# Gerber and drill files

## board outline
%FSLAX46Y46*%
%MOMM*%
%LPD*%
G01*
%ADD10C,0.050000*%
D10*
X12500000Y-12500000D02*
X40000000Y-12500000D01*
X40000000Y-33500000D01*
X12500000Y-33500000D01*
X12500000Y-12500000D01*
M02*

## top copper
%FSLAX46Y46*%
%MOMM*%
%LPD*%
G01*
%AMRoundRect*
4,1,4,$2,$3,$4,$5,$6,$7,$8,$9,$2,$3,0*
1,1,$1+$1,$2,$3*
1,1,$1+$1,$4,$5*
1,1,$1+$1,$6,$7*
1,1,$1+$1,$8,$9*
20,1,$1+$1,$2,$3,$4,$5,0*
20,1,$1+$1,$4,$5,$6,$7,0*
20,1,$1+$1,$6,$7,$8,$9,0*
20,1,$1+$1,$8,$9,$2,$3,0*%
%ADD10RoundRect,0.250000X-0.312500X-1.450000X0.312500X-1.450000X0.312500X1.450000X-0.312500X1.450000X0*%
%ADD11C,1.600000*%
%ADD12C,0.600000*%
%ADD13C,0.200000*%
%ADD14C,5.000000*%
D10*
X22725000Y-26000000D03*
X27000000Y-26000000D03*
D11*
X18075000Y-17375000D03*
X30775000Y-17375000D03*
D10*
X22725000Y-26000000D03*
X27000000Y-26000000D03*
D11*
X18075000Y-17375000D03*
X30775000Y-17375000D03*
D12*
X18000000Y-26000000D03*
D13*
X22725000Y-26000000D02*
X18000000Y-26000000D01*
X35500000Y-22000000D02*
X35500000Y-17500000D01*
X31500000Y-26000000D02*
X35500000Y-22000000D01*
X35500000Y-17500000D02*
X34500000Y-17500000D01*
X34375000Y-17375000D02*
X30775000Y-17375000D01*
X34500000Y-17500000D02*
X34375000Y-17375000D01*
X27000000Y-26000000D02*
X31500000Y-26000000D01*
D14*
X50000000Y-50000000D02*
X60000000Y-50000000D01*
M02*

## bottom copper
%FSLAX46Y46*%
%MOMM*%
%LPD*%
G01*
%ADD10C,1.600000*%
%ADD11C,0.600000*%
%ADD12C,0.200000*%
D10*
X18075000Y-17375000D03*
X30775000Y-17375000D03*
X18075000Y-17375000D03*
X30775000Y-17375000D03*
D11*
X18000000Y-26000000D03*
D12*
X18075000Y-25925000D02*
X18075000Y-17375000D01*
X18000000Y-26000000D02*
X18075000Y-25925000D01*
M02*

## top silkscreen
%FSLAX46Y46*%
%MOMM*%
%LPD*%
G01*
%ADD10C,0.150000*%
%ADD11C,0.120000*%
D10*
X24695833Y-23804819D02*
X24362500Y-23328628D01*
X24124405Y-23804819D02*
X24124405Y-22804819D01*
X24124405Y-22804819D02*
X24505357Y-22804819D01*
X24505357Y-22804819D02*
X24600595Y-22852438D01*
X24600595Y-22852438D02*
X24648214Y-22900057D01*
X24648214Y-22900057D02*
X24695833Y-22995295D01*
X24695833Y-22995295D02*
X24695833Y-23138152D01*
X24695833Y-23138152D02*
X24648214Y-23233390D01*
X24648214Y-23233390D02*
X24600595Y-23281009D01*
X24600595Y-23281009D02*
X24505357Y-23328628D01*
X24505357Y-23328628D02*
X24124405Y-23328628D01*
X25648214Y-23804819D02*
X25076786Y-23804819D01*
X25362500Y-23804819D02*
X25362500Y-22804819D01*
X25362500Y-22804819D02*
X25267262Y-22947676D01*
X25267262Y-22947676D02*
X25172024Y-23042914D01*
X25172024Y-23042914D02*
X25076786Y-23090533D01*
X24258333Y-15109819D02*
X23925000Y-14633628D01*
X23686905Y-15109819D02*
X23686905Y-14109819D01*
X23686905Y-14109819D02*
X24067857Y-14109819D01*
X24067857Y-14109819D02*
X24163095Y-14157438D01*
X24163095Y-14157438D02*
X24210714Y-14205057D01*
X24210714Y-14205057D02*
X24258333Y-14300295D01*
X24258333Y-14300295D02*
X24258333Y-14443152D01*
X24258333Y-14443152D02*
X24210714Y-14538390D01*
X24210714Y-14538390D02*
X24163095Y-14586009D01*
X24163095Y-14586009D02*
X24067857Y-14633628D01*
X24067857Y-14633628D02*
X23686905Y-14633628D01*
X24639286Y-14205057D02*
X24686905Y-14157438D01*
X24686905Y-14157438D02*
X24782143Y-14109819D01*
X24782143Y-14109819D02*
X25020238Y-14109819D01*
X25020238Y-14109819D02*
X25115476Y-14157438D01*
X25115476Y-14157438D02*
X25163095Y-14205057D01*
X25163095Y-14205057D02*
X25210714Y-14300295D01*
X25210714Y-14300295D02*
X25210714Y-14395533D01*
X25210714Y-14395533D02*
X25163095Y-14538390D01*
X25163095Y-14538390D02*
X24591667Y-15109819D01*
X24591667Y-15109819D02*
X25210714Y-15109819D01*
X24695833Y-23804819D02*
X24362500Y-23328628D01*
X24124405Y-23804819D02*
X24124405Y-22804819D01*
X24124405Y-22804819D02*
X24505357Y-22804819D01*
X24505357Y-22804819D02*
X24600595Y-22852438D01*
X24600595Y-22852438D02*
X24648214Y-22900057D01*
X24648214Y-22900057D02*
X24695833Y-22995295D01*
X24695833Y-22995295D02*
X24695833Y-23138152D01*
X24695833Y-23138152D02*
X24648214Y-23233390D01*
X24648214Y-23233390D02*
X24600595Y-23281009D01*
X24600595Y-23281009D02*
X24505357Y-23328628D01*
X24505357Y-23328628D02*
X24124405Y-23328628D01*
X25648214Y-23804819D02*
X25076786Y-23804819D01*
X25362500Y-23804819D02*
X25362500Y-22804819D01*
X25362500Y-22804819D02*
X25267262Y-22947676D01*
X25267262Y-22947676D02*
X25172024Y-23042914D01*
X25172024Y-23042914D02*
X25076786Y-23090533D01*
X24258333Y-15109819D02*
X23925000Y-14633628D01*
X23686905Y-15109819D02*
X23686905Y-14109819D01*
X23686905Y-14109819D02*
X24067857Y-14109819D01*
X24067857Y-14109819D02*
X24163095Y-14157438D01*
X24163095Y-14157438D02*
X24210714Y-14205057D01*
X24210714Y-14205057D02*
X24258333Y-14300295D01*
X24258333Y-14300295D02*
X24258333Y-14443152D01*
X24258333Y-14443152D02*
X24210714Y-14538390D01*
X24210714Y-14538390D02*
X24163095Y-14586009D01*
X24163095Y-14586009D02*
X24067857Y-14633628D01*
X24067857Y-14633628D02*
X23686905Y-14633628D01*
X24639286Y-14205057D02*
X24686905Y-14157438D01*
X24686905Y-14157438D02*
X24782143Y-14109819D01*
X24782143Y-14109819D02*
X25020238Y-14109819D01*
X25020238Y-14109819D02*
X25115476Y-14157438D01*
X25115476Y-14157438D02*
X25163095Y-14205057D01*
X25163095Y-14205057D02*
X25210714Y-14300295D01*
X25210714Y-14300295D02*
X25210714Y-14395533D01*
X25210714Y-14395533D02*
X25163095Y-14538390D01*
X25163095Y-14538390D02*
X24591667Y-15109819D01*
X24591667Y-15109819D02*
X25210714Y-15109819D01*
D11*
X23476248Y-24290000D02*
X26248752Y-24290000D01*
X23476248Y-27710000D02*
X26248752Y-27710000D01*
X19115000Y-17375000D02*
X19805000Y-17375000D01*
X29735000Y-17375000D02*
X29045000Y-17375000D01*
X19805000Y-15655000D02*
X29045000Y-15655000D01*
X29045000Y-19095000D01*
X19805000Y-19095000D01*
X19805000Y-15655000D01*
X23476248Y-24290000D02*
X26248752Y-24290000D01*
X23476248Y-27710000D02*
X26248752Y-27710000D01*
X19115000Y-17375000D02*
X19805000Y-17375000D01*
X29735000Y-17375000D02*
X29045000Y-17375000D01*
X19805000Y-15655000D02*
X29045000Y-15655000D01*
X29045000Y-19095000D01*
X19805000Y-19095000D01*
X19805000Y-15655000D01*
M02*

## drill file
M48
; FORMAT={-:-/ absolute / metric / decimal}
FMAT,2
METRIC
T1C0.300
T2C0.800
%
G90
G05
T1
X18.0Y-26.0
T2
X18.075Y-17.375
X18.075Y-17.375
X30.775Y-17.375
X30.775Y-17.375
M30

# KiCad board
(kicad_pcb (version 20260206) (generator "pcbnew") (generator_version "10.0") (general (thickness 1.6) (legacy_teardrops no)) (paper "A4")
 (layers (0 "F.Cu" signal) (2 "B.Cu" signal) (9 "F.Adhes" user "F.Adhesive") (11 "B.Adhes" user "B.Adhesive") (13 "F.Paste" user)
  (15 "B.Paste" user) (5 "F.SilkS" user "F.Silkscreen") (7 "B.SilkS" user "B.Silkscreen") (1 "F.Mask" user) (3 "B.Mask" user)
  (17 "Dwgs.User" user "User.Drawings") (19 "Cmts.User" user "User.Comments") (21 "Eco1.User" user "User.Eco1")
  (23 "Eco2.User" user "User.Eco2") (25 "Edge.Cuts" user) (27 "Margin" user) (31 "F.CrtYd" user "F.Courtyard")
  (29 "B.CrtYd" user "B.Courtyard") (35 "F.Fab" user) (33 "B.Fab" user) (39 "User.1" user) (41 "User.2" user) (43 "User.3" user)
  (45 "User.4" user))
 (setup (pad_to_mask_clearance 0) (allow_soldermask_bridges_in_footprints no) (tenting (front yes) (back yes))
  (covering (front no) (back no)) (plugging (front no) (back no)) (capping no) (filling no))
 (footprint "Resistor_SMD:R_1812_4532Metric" (layer "F.Cu") (at 24.8625 26)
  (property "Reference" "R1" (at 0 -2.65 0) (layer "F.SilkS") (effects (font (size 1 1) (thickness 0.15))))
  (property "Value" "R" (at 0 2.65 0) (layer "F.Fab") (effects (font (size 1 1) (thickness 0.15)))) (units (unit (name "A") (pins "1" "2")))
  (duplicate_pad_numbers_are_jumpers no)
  (fp_line (start -1.386252 -1.71) (end 1.386252 -1.71) (stroke (width 0.12) (type solid)) (layer "F.SilkS"))
  (fp_line (start -1.386252 1.71) (end 1.386252 1.71) (stroke (width 0.12) (type solid)) (layer "F.SilkS"))
  (pad "1" smd roundrect (at -2.1375 0) (size 1.125 3.4) (layers "F.Cu" "F.Mask" "F.Paste") (roundrect_rratio 0.222222)
   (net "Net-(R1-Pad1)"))
  (pad "2" smd roundrect (at 2.1375 0) (size 1.125 3.4) (layers "F.Cu" "F.Mask" "F.Paste") (roundrect_rratio 0.222222) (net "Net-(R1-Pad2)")))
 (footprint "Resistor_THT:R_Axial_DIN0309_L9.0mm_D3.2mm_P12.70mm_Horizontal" (layer "F.Cu") (at 18.075 17.375)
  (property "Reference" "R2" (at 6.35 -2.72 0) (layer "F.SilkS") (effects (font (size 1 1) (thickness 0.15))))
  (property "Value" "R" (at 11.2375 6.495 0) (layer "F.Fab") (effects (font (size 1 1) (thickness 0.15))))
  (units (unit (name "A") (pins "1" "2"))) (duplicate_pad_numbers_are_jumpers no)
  (fp_line (start 1.04 0) (end 1.73 0) (stroke (width 0.12) (type solid)) (layer "F.SilkS"))
  (fp_line (start 11.66 0) (end 10.97 0) (stroke (width 0.12) (type solid)) (layer "F.SilkS"))
  (fp_rect (start 1.73 -1.72) (end 10.97 1.72) (stroke (width 0.12) (type solid)) (fill no) (layer "F.SilkS"))
  (pad "1" thru_hole circle (at 0 0) (size 1.6 1.6) (drill 0.8) (layers "*.Cu" "*.Mask") (remove_unused_layers no) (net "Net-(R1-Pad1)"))
  (pad "2" thru_hole circle (at 12.7 0) (size 1.6 1.6) (drill 0.8) (layers "*.Cu" "*.Mask") (remove_unused_layers no) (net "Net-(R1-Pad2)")))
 (gr_rect (start 12.5 12.5) (end 40 33.5) (stroke (width 0.05) (type default)) (fill no) (layer "Edge.Cuts"))
 (segment (start 22.725 26) (end 18 26) (width 0.2) (layer "F.Cu") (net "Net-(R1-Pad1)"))
 (segment (start 18.075 25.925) (end 18.075 17.375) (width 0.2) (layer "B.Cu") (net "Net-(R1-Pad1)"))
 (segment (start 18 26) (end 18.075 25.925) (width 0.2) (layer "B.Cu") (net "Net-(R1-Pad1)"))
 (segment (start 35.5 22) (end 35.5 17.5) (width 0.2) (layer "F.Cu") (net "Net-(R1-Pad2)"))
 (segment (start 31.5 26) (end 35.5 22) (width 0.2) (layer "F.Cu") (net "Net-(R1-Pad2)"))
 (segment (start 35.5 17.5) (end 34.5 17.5) (width 0.2) (layer "F.Cu") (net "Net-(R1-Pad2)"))
 (segment (start 34.375 17.375) (end 30.775 17.375) (width 0.2) (layer "F.Cu") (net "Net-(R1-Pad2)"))
 (segment (start 34.5 17.5) (end 34.375 17.375) (width 0.2) (layer "F.Cu") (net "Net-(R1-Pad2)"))
 (segment (start 27 26) (end 31.5 26) (width 0.2) (layer "F.Cu") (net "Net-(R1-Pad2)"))
 (segment (start 50 50) (end 60 50) (width 0.2) (width 5.0) (layer "F.Cu") (layer F.Cu) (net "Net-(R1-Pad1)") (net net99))
 (via (at 18 26) (size 0.6) (drill 0.3) (layers "F.Cu" "B.Cu") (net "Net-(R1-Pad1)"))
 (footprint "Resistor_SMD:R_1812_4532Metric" (layer "F.Cu") (at 24.8625 26)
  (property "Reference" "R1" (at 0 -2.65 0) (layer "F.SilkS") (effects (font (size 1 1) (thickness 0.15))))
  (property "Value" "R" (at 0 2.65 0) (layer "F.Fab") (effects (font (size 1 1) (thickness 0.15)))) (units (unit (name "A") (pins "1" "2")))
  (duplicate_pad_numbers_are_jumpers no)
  (fp_line (start -1.386252 -1.71) (end 1.386252 -1.71) (stroke (width 0.12) (type solid)) (layer "F.SilkS"))
  (fp_line (start -1.386252 1.71) (end 1.386252 1.71) (stroke (width 0.12) (type solid)) (layer "F.SilkS"))
  (pad "1" smd roundrect (at -2.1375 0) (size 1.125 3.4) (layers "F.Cu" "F.Mask" "F.Paste") (roundrect_rratio 0.222222)
   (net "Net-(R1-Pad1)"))
  (pad "2" smd roundrect (at 2.1375 0) (size 1.125 3.4) (layers "F.Cu" "F.Mask" "F.Paste") (roundrect_rratio 0.222222) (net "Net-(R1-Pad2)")))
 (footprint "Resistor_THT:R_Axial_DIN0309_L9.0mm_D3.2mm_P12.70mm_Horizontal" (layer "F.Cu") (at 18.075 17.375)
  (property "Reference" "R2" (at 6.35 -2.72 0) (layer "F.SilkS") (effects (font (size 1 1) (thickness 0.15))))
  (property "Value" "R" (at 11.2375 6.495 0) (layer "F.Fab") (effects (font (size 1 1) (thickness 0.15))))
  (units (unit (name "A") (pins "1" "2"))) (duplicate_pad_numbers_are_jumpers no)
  (fp_line (start 1.04 0) (end 1.73 0) (stroke (width 0.12) (type solid)) (layer "F.SilkS"))
  (fp_line (start 11.66 0) (end 10.97 0) (stroke (width 0.12) (type solid)) (layer "F.SilkS"))
  (fp_rect (start 1.73 -1.72) (end 10.97 1.72) (stroke (width 0.12) (type solid)) (fill no) (layer "F.SilkS"))
  (pad "1" thru_hole circle (at 0 0) (size 1.6 1.6) (drill 0.8) (layers "*.Cu" "*.Mask") (remove_unused_layers no) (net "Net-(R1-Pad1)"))
  (pad "2" thru_hole circle (at 12.7 0) (size 1.6 1.6) (drill 0.8) (layers "*.Cu" "*.Mask") (remove_unused_layers no) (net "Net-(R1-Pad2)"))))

